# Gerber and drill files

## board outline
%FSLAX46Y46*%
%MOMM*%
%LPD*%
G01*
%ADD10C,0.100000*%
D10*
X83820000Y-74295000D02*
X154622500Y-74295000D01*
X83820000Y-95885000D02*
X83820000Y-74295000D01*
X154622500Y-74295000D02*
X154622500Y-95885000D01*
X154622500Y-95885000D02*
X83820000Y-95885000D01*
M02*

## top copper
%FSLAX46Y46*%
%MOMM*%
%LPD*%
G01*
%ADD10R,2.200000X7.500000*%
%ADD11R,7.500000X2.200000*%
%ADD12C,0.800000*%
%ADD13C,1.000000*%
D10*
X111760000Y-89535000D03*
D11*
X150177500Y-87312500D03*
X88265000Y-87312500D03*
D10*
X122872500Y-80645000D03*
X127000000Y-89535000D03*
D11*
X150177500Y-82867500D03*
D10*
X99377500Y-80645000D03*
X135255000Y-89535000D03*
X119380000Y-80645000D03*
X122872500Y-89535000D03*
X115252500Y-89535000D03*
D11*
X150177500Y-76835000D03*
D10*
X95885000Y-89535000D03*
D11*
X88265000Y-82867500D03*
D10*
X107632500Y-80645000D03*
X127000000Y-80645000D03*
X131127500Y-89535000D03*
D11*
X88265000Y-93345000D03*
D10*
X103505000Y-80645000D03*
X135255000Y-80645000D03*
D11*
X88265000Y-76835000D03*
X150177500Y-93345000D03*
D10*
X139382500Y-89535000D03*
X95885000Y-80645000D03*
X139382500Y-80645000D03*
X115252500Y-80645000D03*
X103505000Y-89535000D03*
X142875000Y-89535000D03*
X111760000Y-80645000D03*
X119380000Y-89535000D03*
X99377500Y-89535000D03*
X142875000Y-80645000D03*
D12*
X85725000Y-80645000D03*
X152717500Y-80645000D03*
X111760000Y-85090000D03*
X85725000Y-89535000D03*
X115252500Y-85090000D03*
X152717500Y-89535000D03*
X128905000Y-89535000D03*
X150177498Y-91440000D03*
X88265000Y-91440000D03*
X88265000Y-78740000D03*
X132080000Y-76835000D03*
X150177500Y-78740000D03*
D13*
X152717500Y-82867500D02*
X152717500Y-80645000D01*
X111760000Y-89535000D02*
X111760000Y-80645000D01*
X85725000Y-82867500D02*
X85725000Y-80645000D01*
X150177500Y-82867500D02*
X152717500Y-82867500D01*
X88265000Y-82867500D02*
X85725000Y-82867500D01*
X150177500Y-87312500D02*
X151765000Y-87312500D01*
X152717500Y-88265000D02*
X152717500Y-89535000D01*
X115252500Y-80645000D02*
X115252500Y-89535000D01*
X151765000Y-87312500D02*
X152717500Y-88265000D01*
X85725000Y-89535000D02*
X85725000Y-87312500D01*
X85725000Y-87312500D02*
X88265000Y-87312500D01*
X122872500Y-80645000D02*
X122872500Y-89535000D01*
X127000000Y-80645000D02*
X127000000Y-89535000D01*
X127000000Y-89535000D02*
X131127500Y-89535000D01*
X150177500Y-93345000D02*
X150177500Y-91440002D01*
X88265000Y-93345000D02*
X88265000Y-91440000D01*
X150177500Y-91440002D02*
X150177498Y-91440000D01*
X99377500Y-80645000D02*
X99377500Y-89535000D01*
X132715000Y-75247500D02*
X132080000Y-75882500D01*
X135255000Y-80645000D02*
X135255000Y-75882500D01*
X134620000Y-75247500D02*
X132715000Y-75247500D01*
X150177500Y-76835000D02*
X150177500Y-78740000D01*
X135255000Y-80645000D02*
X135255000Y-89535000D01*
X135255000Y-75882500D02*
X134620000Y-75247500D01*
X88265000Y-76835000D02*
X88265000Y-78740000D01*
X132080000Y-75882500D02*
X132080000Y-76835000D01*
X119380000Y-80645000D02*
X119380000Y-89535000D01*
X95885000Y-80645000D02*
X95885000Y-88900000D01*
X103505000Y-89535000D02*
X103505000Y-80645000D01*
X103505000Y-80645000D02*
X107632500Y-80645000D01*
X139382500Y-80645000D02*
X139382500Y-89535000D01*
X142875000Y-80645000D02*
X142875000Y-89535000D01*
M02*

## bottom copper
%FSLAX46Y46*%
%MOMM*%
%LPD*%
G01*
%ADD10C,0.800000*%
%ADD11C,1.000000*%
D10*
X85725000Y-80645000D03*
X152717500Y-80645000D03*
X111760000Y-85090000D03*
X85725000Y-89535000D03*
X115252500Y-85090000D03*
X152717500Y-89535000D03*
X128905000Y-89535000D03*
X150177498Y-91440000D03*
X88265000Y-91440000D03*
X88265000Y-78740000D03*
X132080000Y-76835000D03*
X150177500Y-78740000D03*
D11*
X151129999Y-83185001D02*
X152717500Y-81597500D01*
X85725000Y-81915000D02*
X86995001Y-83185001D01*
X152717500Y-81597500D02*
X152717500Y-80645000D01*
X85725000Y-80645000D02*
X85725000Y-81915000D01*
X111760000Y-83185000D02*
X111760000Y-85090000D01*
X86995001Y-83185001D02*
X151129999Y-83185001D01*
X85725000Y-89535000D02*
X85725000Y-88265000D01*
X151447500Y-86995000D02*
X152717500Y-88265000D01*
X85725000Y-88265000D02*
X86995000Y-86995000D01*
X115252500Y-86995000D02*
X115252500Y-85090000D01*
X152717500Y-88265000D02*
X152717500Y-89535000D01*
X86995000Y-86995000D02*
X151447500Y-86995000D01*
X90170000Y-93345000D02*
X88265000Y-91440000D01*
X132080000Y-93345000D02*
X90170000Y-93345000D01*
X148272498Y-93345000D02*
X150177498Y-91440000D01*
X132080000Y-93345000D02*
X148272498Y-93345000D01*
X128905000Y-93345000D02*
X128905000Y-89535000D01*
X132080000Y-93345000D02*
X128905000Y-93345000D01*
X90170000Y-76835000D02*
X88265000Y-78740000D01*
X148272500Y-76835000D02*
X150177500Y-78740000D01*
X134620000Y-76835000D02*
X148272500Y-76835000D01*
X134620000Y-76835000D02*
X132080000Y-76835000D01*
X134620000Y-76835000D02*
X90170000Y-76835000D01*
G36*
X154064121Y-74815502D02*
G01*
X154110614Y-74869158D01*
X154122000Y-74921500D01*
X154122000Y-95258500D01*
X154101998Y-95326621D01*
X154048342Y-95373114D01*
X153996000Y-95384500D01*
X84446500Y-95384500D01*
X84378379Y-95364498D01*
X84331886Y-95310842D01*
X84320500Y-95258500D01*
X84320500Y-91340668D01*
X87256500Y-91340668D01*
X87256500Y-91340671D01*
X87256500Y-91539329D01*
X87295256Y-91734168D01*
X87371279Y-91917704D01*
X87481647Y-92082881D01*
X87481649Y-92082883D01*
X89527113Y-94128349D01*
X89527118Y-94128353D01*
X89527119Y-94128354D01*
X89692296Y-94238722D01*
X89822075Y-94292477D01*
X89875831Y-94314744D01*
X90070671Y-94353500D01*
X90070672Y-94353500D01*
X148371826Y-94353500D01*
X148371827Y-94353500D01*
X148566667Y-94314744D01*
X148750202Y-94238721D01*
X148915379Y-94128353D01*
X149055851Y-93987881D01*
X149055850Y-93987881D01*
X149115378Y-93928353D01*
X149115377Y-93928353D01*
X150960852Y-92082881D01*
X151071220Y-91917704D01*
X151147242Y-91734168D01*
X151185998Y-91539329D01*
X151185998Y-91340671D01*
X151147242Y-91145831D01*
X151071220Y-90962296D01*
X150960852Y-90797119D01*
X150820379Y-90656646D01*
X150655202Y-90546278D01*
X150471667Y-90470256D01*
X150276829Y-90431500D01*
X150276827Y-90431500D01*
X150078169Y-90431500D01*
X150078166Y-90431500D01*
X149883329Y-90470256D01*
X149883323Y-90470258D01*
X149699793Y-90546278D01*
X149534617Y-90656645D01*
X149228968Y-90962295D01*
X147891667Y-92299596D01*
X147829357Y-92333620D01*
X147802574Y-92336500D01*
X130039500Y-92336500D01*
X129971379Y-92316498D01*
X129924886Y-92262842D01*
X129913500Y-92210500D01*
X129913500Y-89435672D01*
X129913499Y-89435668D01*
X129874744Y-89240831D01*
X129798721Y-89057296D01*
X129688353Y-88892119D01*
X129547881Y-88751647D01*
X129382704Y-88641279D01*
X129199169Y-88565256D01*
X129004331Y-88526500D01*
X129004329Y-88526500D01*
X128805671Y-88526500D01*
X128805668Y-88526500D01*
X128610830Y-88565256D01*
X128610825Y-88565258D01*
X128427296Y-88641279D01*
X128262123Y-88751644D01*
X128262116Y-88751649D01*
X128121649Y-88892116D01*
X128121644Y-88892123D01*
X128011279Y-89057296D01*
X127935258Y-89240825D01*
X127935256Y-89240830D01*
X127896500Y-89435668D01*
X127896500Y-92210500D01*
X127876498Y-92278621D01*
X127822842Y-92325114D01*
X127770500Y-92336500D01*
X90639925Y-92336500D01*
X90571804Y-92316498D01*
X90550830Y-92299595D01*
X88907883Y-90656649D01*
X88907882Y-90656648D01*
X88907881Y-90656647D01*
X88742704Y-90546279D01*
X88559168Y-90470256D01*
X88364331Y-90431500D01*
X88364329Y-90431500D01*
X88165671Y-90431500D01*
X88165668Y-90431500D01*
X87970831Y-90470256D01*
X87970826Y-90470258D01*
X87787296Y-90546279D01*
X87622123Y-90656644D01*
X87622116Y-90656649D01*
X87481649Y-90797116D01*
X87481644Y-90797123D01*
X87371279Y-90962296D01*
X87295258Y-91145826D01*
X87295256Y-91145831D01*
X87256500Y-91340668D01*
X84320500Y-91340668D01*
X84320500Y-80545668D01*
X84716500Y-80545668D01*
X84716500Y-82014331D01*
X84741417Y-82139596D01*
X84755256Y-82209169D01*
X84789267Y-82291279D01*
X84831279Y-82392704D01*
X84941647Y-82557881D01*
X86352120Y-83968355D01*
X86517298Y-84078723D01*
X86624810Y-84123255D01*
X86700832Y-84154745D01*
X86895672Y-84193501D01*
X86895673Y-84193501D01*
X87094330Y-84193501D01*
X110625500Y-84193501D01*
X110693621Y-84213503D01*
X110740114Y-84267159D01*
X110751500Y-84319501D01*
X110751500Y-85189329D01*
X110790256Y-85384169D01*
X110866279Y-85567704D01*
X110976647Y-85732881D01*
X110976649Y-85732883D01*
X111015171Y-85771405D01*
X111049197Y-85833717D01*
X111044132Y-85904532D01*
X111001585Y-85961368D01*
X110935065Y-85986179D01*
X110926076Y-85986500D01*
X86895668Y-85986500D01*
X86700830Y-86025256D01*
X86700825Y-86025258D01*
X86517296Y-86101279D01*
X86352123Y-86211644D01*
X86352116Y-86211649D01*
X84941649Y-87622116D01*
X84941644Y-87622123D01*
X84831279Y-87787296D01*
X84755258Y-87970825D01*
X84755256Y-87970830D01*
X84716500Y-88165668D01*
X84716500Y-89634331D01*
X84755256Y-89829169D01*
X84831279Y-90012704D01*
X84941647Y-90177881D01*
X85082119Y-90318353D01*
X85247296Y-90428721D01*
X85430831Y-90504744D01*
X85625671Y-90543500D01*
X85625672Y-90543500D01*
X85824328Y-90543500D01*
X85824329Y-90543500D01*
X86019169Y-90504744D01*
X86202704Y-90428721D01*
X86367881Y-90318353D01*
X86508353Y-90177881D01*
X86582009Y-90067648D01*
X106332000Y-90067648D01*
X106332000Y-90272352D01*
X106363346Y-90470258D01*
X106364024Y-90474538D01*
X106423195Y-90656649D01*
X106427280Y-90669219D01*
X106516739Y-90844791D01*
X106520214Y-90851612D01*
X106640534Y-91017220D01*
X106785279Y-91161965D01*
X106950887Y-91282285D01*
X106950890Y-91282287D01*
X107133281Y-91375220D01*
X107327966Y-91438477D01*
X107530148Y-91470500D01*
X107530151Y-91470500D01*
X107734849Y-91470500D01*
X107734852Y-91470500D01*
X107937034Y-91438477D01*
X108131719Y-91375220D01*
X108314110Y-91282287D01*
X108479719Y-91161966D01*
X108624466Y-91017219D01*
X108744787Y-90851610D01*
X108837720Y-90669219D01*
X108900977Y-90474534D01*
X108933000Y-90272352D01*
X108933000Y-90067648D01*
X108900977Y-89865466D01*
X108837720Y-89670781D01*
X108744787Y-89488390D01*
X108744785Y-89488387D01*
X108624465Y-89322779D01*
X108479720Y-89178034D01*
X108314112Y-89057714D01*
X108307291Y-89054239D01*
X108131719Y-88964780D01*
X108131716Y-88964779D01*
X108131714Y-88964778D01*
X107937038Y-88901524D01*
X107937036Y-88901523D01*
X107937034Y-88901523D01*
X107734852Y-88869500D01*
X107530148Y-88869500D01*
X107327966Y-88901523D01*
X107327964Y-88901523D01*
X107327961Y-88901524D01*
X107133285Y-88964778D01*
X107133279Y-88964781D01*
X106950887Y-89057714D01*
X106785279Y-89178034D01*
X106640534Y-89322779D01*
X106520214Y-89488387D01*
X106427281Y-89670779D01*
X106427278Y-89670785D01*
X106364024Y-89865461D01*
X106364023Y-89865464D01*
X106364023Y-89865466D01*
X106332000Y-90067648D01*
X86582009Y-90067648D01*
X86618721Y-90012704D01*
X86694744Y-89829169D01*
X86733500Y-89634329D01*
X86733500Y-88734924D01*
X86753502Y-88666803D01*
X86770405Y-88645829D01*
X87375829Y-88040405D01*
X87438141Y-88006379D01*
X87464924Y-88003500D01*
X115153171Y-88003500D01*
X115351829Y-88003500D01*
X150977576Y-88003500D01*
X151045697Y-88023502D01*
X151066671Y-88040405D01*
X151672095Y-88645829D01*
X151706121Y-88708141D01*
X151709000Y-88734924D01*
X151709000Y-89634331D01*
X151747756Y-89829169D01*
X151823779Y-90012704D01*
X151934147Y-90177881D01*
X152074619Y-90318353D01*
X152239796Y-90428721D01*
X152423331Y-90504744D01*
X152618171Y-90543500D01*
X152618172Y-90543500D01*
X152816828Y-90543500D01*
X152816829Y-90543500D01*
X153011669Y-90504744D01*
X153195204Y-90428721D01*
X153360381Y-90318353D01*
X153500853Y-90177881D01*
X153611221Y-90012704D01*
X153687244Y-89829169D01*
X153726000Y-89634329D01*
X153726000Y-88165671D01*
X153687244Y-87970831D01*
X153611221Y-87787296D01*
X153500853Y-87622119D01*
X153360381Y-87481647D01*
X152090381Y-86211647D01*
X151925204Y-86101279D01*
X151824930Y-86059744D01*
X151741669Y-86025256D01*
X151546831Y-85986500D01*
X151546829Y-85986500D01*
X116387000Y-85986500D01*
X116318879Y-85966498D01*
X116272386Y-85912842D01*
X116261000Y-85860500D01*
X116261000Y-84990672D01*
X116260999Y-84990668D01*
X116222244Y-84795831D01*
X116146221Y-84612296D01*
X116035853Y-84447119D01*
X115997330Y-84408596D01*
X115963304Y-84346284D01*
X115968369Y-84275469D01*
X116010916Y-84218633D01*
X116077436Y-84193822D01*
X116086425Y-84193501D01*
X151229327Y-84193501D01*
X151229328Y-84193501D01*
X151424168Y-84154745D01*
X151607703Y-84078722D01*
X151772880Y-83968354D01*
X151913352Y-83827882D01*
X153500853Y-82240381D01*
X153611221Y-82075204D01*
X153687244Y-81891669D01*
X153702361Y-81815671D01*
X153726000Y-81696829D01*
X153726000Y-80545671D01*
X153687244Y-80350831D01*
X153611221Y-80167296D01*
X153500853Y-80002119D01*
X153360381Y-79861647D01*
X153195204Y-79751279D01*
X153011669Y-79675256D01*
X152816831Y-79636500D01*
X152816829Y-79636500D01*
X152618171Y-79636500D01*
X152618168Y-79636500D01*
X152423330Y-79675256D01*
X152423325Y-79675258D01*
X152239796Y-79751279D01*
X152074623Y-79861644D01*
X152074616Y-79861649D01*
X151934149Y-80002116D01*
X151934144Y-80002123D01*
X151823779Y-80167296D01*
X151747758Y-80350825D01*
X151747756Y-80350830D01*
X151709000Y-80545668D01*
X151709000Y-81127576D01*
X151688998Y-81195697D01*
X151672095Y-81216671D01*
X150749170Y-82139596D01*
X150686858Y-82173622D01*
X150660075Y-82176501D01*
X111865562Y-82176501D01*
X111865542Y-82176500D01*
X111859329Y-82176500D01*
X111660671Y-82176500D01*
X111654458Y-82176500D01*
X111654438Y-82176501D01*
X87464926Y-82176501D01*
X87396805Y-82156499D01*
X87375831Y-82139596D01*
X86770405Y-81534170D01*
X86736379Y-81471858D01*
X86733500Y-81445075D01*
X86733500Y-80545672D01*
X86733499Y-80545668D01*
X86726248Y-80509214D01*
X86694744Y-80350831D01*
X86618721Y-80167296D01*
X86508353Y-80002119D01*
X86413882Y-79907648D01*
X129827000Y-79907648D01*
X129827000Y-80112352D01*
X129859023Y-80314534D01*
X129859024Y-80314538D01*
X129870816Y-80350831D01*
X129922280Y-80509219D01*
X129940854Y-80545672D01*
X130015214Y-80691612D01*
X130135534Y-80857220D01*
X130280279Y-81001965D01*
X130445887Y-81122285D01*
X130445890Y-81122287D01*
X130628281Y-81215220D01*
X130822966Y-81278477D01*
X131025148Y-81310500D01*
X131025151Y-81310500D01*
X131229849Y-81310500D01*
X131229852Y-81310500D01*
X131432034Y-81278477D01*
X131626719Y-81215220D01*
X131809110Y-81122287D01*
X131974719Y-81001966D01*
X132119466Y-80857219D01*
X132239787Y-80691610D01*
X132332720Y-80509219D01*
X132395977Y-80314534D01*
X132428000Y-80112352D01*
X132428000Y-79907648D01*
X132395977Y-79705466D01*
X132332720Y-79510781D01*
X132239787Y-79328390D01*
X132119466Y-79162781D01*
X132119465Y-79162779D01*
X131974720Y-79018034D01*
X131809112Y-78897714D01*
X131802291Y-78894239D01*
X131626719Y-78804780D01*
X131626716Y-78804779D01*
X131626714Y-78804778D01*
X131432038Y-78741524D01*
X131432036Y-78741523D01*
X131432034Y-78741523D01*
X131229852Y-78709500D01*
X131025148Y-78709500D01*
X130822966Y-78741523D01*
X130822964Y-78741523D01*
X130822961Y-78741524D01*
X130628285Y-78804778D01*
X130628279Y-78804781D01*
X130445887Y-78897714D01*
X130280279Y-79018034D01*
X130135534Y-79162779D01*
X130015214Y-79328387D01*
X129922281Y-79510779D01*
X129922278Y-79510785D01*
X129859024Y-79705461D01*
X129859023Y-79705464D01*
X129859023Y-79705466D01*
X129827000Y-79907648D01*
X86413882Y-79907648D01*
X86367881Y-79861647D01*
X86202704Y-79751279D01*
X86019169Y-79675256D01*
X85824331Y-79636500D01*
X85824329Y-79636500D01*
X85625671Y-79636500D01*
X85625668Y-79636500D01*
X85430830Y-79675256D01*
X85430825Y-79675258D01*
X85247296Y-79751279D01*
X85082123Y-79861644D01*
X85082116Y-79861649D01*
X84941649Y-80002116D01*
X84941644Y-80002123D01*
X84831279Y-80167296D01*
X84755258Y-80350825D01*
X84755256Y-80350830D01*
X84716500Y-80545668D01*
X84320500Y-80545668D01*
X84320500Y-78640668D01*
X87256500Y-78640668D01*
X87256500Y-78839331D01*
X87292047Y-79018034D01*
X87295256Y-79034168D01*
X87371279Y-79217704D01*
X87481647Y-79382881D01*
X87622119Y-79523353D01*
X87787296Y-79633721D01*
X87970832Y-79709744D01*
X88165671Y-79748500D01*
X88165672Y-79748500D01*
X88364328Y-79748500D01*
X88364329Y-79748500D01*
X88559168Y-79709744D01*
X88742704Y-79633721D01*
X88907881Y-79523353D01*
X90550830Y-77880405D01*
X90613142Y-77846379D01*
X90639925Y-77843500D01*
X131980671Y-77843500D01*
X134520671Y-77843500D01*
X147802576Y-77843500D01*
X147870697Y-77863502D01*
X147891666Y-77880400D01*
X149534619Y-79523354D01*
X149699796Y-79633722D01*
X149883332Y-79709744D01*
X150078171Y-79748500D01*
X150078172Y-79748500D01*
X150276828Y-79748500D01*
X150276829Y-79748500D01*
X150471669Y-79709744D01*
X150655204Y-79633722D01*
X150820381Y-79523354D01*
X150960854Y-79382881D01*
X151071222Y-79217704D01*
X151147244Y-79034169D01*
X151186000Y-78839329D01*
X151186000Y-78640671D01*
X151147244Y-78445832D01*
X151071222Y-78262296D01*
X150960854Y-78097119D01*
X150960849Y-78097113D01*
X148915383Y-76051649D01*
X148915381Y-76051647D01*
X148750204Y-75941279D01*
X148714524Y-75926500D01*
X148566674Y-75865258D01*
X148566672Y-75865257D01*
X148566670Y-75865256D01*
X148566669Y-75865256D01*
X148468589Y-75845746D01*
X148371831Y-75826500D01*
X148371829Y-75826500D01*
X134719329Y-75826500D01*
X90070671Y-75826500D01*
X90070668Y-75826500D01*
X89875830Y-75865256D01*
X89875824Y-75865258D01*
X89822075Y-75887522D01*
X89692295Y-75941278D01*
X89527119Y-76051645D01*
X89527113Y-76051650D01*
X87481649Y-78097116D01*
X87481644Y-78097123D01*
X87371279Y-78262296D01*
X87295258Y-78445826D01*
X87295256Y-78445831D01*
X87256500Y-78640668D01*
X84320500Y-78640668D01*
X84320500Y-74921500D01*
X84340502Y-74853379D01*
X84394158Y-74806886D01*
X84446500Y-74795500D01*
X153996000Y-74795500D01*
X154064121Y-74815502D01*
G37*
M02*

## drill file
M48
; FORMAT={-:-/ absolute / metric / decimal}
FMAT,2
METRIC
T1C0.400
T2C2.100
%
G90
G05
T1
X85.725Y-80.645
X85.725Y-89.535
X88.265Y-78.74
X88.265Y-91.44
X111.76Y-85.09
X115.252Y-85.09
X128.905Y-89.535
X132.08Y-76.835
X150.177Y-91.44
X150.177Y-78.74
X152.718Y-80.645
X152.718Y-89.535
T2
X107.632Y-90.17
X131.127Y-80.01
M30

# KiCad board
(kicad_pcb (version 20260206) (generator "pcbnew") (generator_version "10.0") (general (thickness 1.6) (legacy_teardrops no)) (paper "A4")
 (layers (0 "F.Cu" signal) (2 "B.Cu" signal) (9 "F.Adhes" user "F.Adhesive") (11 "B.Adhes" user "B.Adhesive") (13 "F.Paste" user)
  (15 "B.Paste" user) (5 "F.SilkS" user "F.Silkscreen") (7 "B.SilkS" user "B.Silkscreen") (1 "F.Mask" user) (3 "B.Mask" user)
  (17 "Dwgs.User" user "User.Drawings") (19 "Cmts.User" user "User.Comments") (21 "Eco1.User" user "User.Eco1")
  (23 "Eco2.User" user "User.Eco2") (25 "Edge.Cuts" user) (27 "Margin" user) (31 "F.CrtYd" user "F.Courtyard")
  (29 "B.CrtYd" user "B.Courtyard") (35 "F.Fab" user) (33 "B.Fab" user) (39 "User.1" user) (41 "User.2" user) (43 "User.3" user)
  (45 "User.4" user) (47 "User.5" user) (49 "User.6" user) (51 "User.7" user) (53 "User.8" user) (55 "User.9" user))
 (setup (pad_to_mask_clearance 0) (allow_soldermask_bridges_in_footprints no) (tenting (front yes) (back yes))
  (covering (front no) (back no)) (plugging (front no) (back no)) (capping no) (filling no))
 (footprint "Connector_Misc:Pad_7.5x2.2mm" (layer "F.Cu") (at 111.76 89.535 -90)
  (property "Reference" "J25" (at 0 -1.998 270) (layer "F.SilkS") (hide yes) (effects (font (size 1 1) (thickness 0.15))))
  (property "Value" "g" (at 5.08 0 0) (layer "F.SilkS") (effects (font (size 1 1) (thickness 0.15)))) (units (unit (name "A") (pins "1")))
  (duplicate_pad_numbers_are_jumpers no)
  (pad "1" smd rect (at 0 0 270) (size 7.5 2.2) (layers "F.Cu" "F.Mask") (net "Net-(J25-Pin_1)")))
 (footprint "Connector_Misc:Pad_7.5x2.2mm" (layer "F.Cu") (at 150.1775 87.3125)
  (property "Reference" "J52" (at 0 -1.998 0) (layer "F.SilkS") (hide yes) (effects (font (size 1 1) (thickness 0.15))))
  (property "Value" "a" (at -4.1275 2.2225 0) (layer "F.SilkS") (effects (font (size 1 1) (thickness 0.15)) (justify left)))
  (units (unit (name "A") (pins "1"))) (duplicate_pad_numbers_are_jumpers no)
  (pad "1" smd rect (at 0 0) (size 7.5 2.2) (layers "F.Cu" "F.Mask") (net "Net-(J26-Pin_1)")))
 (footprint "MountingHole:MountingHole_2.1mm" (layer "F.Cu") (at 107.6325 90.17)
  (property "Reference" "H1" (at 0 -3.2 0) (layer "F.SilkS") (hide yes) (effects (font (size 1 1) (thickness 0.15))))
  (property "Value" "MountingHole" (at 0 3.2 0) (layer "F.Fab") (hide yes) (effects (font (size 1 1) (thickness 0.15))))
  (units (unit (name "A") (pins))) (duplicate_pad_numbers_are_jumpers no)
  (pad "" np_thru_hole circle (at 0 0) (size 2.1 2.1) (drill 2.1) (layers "*.Cu" "*.Mask")))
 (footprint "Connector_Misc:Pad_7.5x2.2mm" (layer "F.Cu") (at 88.265 87.3125 180)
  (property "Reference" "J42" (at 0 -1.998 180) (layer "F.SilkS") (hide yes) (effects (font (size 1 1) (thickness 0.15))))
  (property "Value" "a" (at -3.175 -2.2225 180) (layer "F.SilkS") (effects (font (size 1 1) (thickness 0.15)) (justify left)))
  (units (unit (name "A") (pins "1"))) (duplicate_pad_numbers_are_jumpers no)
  (pad "1" smd rect (at 0 0 180) (size 7.5 2.2) (layers "F.Cu" "F.Mask") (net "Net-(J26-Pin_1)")))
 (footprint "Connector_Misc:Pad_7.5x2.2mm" (layer "F.Cu") (at 122.8725 80.645 90)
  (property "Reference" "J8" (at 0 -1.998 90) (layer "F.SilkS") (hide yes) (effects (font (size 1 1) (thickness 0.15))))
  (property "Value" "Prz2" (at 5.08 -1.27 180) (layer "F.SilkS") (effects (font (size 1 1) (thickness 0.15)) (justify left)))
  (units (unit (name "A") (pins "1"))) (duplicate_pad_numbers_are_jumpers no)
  (pad "1" smd rect (at 0 0 90) (size 7.5 2.2) (layers "F.Cu" "F.Mask") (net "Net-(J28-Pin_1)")))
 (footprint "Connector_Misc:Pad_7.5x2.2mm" (layer "F.Cu") (at 127 89.535 -90)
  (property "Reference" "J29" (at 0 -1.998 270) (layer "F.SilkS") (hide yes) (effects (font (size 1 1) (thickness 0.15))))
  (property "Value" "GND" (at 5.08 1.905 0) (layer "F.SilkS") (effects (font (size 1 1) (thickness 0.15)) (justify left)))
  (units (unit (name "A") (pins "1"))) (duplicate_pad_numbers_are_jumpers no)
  (pad "1" smd rect (at 0 0 270) (size 7.5 2.2) (layers "F.Cu" "F.Mask") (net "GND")))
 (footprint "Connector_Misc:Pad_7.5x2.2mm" (layer "F.Cu") (at 150.1775 82.8675)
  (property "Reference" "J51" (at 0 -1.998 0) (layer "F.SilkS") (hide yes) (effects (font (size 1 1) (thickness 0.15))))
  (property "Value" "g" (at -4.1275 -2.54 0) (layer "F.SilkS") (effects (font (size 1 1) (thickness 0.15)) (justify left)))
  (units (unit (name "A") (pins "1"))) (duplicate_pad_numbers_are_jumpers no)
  (pad "1" smd rect (at 0 0) (size 7.5 2.2) (layers "F.Cu" "F.Mask") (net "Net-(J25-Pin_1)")))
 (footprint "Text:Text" (layer "F.Cu") (at 102.743 79.883)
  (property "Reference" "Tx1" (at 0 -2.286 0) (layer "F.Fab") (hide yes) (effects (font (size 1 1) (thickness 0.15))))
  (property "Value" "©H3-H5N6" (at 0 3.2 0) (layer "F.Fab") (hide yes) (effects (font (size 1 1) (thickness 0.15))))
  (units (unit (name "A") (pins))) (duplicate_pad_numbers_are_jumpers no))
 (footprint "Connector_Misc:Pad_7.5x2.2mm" (layer "F.Cu") (at 99.3775 80.645 90)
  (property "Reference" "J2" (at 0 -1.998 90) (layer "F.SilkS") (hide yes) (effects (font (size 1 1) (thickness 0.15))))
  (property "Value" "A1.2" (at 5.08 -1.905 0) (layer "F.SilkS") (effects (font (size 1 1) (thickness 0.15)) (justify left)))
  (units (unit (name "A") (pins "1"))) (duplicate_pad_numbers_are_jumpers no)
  (pad "1" smd rect (at 0 0 90) (size 7.5 2.2) (layers "F.Cu" "F.Mask") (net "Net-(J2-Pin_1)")))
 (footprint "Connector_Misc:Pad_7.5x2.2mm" (layer "F.Cu") (at 135.255 89.535 90)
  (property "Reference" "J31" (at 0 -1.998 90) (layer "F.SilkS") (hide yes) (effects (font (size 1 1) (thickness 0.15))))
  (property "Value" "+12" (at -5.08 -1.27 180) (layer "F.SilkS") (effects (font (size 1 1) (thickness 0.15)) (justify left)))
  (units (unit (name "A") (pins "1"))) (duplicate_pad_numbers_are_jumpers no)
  (pad "1" smd rect (at 0 0 90) (size 7.5 2.2) (layers "F.Cu" "F.Mask") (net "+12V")))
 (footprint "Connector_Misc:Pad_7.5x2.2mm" (layer "F.Cu") (at 119.38 80.645 90)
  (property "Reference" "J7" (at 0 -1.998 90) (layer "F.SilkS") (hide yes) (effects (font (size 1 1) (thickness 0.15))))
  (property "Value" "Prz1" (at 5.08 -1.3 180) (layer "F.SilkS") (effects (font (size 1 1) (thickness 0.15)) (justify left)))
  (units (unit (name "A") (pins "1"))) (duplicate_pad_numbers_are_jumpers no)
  (pad "1" smd rect (at 0 0 90) (size 7.5 2.2) (layers "F.Cu" "F.Mask") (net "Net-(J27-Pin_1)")))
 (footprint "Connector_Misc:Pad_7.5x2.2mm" (layer "F.Cu") (at 122.8725 89.535 -90)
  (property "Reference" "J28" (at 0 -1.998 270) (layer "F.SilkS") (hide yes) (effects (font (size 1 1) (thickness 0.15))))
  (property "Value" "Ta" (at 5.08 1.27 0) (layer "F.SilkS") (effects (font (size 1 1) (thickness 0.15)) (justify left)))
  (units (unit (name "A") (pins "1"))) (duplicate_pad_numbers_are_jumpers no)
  (pad "1" smd rect (at 0 0 270) (size 7.5 2.2) (layers "F.Cu" "F.Mask") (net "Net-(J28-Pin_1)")))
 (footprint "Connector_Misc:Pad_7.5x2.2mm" (layer "F.Cu") (at 115.2525 89.535 -90)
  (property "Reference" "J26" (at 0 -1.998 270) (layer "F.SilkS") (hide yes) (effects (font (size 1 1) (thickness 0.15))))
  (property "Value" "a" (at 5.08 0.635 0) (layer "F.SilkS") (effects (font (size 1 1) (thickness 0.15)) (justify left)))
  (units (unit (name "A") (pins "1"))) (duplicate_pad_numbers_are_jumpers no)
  (pad "1" smd rect (at 0 0 270) (size 7.5 2.2) (layers "F.Cu" "F.Mask") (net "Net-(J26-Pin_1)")))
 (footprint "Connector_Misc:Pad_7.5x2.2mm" (layer "F.Cu") (at 150.1775 76.835 180)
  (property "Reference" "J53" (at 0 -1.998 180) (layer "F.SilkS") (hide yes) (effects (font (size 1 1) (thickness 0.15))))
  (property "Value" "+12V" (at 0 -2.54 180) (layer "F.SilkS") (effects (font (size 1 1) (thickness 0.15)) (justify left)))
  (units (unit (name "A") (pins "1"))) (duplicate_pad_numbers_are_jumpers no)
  (pad "1" smd rect (at 0 0 180) (size 7.5 2.2) (layers "F.Cu" "F.Mask") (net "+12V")))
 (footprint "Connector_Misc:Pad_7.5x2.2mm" (layer "F.Cu") (at 95.885 89.535 -90)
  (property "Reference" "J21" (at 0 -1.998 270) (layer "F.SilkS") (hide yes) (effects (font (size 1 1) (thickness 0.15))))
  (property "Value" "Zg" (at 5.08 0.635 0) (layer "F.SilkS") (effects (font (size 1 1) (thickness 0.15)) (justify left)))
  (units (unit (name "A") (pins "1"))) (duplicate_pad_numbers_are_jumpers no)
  (pad "1" smd rect (at 0 0 270) (size 7.5 2.2) (layers "F.Cu" "F.Mask") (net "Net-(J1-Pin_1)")))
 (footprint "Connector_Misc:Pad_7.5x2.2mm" (layer "F.Cu") (at 88.265 82.8675 180)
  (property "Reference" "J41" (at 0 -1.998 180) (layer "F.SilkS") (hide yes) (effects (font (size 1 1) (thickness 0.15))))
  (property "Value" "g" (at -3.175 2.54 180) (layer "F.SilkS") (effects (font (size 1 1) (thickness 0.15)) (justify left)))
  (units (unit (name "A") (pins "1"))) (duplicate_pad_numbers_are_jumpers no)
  (pad "1" smd rect (at 0 0 180) (size 7.5 2.2) (layers "F.Cu" "F.Mask") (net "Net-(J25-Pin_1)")))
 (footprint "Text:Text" (layer "F.Cu") (at 124.587 89.535)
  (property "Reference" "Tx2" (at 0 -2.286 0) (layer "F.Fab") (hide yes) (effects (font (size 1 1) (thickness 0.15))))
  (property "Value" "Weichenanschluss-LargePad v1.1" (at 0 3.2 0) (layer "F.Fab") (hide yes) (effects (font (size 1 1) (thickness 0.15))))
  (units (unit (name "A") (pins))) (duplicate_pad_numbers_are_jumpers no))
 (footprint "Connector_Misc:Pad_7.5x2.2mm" (layer "F.Cu") (at 107.6325 80.645 90)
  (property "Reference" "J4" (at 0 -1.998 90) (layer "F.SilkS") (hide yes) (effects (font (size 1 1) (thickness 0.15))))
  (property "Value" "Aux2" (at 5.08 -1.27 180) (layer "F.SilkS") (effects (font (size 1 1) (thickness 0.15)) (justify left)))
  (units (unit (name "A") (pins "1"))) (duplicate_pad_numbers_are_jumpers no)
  (pad "1" smd rect (at 0 0 90) (size 7.5 2.2) (layers "F.Cu" "F.Mask") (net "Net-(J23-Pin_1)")))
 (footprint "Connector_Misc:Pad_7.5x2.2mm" (layer "F.Cu") (at 127 80.645 90)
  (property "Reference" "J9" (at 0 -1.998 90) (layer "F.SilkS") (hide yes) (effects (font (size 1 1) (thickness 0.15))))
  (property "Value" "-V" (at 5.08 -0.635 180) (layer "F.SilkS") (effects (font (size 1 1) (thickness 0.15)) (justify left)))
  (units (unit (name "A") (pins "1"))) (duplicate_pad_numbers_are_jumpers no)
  (pad "1" smd rect (at 0 0 90) (size 7.5 2.2) (layers "F.Cu" "F.Mask") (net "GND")))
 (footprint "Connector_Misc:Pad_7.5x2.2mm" (layer "F.Cu") (at 131.1275 89.535 -90)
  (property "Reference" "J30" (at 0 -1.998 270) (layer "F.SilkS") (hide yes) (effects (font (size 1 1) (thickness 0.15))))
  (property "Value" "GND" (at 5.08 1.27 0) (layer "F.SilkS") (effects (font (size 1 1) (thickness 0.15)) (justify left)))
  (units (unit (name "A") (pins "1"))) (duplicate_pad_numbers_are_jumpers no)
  (pad "1" smd rect (at 0 0 270) (size 7.5 2.2) (layers "F.Cu" "F.Mask") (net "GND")))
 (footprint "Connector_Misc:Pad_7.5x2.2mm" (layer "F.Cu") (at 88.265 93.345)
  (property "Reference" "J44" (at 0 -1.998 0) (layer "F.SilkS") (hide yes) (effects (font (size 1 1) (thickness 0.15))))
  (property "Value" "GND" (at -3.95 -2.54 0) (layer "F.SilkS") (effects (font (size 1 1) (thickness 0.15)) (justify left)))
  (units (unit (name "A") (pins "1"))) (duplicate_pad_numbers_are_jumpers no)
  (pad "1" smd rect (at 0 0) (size 7.5 2.2) (layers "F.Cu" "F.Mask") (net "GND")))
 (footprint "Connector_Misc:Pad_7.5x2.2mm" (layer "F.Cu") (at 103.505 80.645 90)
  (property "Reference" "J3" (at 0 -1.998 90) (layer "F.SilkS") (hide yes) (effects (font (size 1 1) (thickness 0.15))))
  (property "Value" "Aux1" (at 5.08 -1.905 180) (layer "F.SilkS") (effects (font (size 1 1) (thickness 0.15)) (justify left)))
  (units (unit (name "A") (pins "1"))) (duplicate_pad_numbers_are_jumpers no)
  (pad "1" smd rect (at 0 0 90) (size 7.5 2.2) (layers "F.Cu" "F.Mask") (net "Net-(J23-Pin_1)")))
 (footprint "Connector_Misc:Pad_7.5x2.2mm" (layer "F.Cu") (at 135.255 80.645 90)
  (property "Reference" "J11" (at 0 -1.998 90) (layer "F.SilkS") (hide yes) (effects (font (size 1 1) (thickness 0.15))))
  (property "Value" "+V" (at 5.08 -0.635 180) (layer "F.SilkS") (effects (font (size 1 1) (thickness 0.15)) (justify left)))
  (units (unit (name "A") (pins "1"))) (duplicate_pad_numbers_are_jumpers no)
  (pad "1" smd rect (at 0 0 90) (size 7.5 2.2) (layers "F.Cu" "F.Mask") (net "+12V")))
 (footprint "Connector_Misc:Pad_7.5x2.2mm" (layer "F.Cu") (at 88.265 76.835)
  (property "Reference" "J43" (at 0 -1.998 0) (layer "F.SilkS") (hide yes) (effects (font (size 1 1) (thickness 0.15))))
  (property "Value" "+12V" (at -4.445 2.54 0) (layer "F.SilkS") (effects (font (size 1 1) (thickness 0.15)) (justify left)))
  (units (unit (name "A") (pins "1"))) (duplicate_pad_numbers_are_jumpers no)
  (pad "1" smd rect (at 0 0) (size 7.5 2.2) (layers "F.Cu" "F.Mask") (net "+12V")))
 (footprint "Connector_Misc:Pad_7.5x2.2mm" (layer "F.Cu") (at 150.1775 93.345)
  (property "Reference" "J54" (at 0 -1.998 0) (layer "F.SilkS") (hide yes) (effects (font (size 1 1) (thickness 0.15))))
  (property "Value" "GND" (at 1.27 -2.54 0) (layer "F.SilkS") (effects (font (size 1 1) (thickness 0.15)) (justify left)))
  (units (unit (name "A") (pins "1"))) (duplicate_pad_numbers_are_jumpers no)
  (pad "1" smd rect (at 0 0) (size 7.5 2.2) (layers "F.Cu" "F.Mask") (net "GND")))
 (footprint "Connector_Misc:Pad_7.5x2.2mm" (layer "F.Cu") (at 139.3825 89.535 90)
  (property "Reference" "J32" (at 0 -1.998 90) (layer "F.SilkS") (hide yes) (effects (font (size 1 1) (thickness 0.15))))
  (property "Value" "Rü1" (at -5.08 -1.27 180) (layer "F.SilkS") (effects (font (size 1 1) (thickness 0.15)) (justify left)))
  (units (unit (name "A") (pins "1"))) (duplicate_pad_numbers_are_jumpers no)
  (pad "1" smd rect (at 0 0 90) (size 7.5 2.2) (layers "F.Cu" "F.Mask") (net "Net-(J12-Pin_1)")))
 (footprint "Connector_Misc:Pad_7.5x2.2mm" (layer "F.Cu") (at 95.885 80.645 90)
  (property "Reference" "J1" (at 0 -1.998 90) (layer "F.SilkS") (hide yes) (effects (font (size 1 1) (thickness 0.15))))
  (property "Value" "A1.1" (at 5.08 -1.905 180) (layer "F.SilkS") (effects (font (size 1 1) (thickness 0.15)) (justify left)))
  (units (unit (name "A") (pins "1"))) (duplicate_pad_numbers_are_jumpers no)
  (pad "1" smd rect (at 0 0 90) (size 7.5 2.2) (layers "F.Cu" "F.Mask") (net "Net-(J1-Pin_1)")))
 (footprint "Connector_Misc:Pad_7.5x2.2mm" (layer "F.Cu") (at 139.3825 80.645 90)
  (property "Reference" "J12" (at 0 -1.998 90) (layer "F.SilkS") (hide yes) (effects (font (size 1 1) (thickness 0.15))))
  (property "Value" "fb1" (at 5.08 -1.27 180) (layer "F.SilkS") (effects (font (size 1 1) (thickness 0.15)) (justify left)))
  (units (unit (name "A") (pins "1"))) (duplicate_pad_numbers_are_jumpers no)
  (pad "1" smd rect (at 0 0 90) (size 7.5 2.2) (layers "F.Cu" "F.Mask") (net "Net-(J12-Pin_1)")))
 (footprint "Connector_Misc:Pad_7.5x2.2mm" (layer "F.Cu") (at 115.2525 80.645 90)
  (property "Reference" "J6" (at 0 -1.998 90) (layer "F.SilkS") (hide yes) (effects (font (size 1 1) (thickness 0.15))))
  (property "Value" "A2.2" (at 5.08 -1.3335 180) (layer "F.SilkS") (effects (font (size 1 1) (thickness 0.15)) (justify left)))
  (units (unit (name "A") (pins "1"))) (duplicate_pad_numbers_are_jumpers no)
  (pad "1" smd rect (at 0 0 90) (size 7.5 2.2) (layers "F.Cu" "F.Mask") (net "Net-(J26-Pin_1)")))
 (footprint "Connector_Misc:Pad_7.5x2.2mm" (layer "F.Cu") (at 103.505 89.535 -90)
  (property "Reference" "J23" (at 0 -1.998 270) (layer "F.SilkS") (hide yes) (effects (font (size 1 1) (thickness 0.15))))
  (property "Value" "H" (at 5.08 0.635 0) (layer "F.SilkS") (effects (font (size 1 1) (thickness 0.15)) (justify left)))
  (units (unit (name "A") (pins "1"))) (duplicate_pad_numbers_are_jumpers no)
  (pad "1" smd rect (at 0 0 270) (size 7.5 2.2) (layers "F.Cu" "F.Mask") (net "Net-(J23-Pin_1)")))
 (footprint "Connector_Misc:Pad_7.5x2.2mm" (layer "F.Cu") (at 142.875 89.535 90)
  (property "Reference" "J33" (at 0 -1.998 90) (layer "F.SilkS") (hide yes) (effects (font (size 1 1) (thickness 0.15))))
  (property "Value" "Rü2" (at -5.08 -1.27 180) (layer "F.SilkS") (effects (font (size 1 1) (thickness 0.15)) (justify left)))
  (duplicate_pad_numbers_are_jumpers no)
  (pad "1" smd rect (at 0 0 90) (size 7.5 2.2) (layers "F.Cu" "F.Mask") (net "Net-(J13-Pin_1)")))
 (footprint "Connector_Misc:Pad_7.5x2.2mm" (layer "F.Cu") (at 111.76 80.645 90)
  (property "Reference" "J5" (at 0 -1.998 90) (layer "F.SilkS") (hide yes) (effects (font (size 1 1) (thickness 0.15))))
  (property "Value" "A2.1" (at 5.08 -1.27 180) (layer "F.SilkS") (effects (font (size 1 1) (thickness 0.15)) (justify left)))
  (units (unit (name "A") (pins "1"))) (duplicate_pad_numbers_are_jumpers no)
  (pad "1" smd rect (at 0 0 90) (size 7.5 2.2) (layers "F.Cu" "F.Mask") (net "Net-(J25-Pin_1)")))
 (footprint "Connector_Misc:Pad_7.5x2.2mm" (layer "F.Cu") (at 119.38 89.535 -90)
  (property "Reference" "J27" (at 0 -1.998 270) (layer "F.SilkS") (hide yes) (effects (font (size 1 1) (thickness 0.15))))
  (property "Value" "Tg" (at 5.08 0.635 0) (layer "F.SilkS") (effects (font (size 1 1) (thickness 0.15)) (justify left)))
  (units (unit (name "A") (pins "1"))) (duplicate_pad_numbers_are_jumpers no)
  (pad "1" smd rect (at 0 0 270) (size 7.5 2.2) (layers "F.Cu" "F.Mask") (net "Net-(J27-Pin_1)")))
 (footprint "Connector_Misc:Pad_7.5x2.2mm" (layer "F.Cu") (at 99.3775 89.535 -90)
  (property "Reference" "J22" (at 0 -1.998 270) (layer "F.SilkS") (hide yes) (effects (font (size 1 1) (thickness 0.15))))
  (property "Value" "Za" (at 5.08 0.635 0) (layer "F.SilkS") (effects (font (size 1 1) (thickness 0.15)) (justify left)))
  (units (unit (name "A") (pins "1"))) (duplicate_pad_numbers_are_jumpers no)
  (pad "1" smd rect (at 0 0 270) (size 7.5 2.2) (layers "F.Cu" "F.Mask") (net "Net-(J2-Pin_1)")))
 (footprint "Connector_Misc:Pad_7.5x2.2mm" (layer "F.Cu") (at 142.875 80.645 90)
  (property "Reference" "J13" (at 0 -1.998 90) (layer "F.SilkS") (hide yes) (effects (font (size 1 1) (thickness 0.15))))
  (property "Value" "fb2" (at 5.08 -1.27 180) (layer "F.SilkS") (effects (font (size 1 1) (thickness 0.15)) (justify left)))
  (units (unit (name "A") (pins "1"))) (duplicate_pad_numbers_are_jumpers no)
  (pad "1" smd rect (at 0 0 90) (size 7.5 2.2) (layers "F.Cu" "F.Mask") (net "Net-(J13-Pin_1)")))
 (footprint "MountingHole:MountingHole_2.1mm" (layer "F.Cu") (at 131.1275 80.01)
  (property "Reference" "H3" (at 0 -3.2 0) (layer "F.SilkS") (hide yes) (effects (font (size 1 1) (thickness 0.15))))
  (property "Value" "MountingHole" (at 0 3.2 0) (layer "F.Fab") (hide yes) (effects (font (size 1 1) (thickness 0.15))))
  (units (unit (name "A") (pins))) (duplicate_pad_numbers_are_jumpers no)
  (pad "" np_thru_hole circle (at 0 0) (size 2.1 2.1) (drill 2.1) (layers "*.Cu" "*.Mask")))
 (gr_line (start 83.82 74.295) (end 154.6225 74.295) (stroke (width 0.1) (type solid)) (layer "Edge.Cuts"))
 (gr_line (start 83.82 95.885) (end 83.82 74.295) (stroke (width 0.1) (type solid)) (layer "Edge.Cuts"))
 (gr_line (start 154.6225 74.295) (end 154.6225 95.885) (stroke (width 0.1) (type solid)) (layer "Edge.Cuts"))
 (gr_line (start 154.6225 95.885) (end 83.82 95.885) (stroke (width 0.1) (type solid)) (layer "Edge.Cuts"))
 (segment (start 152.7175 82.8675) (end 152.7175 80.645) (width 1) (layer "F.Cu") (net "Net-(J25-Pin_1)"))
 (segment (start 111.76 89.535) (end 111.76 80.645) (width 1) (layer "F.Cu") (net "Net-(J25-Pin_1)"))
 (segment (start 85.725 82.8675) (end 85.725 80.645) (width 1) (layer "F.Cu") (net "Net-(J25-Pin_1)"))
 (segment (start 150.1775 82.8675) (end 152.7175 82.8675) (width 1) (layer "F.Cu") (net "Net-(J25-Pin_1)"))
 (segment (start 88.265 82.8675) (end 85.725 82.8675) (width 1) (layer "F.Cu") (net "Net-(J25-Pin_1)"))
 (via (at 85.725 80.645) (size 0.8) (drill 0.4) (layers "F.Cu" "B.Cu") (capping no) (covering (front no) (back no))
  (plugging (front no) (back no)) (filling no) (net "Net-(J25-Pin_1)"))
 (via (at 152.7175 80.645) (size 0.8) (drill 0.4) (layers "F.Cu" "B.Cu") (capping no) (covering (front no) (back no))
  (plugging (front no) (back no)) (filling no) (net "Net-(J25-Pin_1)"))
 (via (at 111.76 85.09) (size 0.8) (drill 0.4) (layers "F.Cu" "B.Cu") (capping no) (covering (front no) (back no))
  (plugging (front no) (back no)) (filling no) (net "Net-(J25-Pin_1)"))
 (segment (start 151.129999 83.185001) (end 152.7175 81.5975) (width 1) (layer "B.Cu") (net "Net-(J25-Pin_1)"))
 (segment (start 85.725 81.915) (end 86.995001 83.185001) (width 1) (layer "B.Cu") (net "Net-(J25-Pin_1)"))
 (segment (start 152.7175 81.5975) (end 152.7175 80.645) (width 1) (layer "B.Cu") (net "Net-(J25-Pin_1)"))
 (segment (start 85.725 80.645) (end 85.725 81.915) (width 1) (layer "B.Cu") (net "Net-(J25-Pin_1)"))
 (segment (start 111.76 83.185) (end 111.76 85.09) (width 1) (layer "B.Cu") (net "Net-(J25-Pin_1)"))
 (segment (start 86.995001 83.185001) (end 151.129999 83.185001) (width 1) (layer "B.Cu") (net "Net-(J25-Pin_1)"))
 (segment (start 150.1775 87.3125) (end 151.765 87.3125) (width 1) (layer "F.Cu") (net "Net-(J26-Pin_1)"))
 (segment (start 152.7175 88.265) (end 152.7175 89.535) (width 1) (layer "F.Cu") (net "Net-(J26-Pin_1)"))
 (segment (start 115.2525 80.645) (end 115.2525 89.535) (width 1) (layer "F.Cu") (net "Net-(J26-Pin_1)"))
 (segment (start 151.765 87.3125) (end 152.7175 88.265) (width 1) (layer "F.Cu") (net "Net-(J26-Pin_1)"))
 (segment (start 85.725 89.535) (end 85.725 87.3125) (width 1) (layer "F.Cu") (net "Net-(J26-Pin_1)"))
 (segment (start 85.725 87.3125) (end 88.265 87.3125) (width 1) (layer "F.Cu") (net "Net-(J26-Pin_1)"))
 (via (at 85.725 89.535) (size 0.8) (drill 0.4) (layers "F.Cu" "B.Cu") (capping no) (covering (front no) (back no))
  (plugging (front no) (back no)) (filling no) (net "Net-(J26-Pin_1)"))
 (via (at 115.2525 85.09) (size 0.8) (drill 0.4) (layers "F.Cu" "B.Cu") (capping no) (covering (front no) (back no))
  (plugging (front no) (back no)) (filling no) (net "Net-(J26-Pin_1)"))
 (via (at 152.7175 89.535) (size 0.8) (drill 0.4) (layers "F.Cu" "B.Cu") (capping no) (covering (front no) (back no))
  (plugging (front no) (back no)) (filling no) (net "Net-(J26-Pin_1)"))
 (segment (start 85.725 89.535) (end 85.725 88.265) (width 1) (layer "B.Cu") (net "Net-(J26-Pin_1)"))
 (segment (start 151.4475 86.995) (end 152.7175 88.265) (width 1) (layer "B.Cu") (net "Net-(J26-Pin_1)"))
 (segment (start 85.725 88.265) (end 86.995 86.995) (width 1) (layer "B.Cu") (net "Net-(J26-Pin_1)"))
 (segment (start 115.2525 86.995) (end 115.2525 85.09) (width 1) (layer "B.Cu") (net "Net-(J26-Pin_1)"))
 (segment (start 152.7175 88.265) (end 152.7175 89.535) (width 1) (layer "B.Cu") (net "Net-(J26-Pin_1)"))
 (segment (start 86.995 86.995) (end 151.4475 86.995) (width 1) (layer "B.Cu") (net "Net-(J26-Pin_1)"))
 (segment (start 122.8725 80.645) (end 122.8725 89.535) (width 1) (layer "F.Cu") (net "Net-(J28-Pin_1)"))
 (segment (start 127 80.645) (end 127 89.535) (width 1) (layer "F.Cu") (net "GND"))
 (segment (start 127 89.535) (end 131.1275 89.535) (width 1) (layer "F.Cu") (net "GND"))
 (segment (start 150.1775 93.345) (end 150.1775 91.440002) (width 1) (layer "F.Cu") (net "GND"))
 (segment (start 88.265 93.345) (end 88.265 91.44) (width 1) (layer "F.Cu") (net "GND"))
 (segment (start 150.1775 91.440002) (end 150.177498 91.44) (width 1) (layer "F.Cu") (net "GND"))
 (via (at 128.905 89.535) (size 0.8) (drill 0.4) (layers "F.Cu" "B.Cu") (capping no) (covering (front no) (back no))
  (plugging (front no) (back no)) (filling no) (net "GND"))
 (via (at 150.177498 91.44) (size 0.8) (drill 0.4) (layers "F.Cu" "B.Cu") (capping no) (covering (front no) (back no))
  (plugging (front no) (back no)) (filling no) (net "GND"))
 (via (at 88.265 91.44) (size 0.8) (drill 0.4) (layers "F.Cu" "B.Cu") (capping no) (covering (front no) (back no))
  (plugging (front no) (back no)) (filling no) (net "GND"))
 (segment (start 90.17 93.345) (end 88.265 91.44) (width 1) (layer "B.Cu") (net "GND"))
 (segment (start 132.08 93.345) (end 90.17 93.345) (width 1) (layer "B.Cu") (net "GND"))
 (segment (start 148.272498 93.345) (end 150.177498 91.44) (width 1) (layer "B.Cu") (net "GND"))
 (segment (start 132.08 93.345) (end 148.272498 93.345) (width 1) (layer "B.Cu") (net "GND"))
 (segment (start 128.905 93.345) (end 128.905 89.535) (width 1) (layer "B.Cu") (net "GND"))
 (segment (start 132.08 93.345) (end 128.905 93.345) (width 1) (layer "B.Cu") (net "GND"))
 (segment (start 99.3775 80.645) (end 99.3775 89.535) (width 1) (layer "F.Cu") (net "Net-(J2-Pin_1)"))
 (segment (start 132.715 75.2475) (end 132.08 75.8825) (width 1) (layer "F.Cu") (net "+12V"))
 (segment (start 135.255 80.645) (end 135.255 75.8825) (width 1) (layer "F.Cu") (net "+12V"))
 (segment (start 134.62 75.2475) (end 132.715 75.2475) (width 1) (layer "F.Cu") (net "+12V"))
 (segment (start 150.1775 76.835) (end 150.1775 78.74) (width 1) (layer "F.Cu") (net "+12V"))
 (segment (start 135.255 80.645) (end 135.255 89.535) (width 1) (layer "F.Cu") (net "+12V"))
 (segment (start 135.255 75.8825) (end 134.62 75.2475) (width 1) (layer "F.Cu") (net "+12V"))
 (segment (start 88.265 76.835) (end 88.265 78.74) (width 1) (layer "F.Cu") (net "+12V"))
 (segment (start 132.08 75.8825) (end 132.08 76.835) (width 1) (layer "F.Cu") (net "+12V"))
 (via (at 88.265 78.74) (size 0.8) (drill 0.4) (layers "F.Cu" "B.Cu") (capping no) (covering (front no) (back no))
  (plugging (front no) (back no)) (filling no) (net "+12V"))
 (via (at 132.08 76.835) (size 0.8) (drill 0.4) (layers "F.Cu" "B.Cu") (capping no) (covering (front no) (back no))
  (plugging (front no) (back no)) (filling no) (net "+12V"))
 (via (at 150.1775 78.74) (size 0.8) (drill 0.4) (layers "F.Cu" "B.Cu") (capping no) (covering (front no) (back no))
  (plugging (front no) (back no)) (filling no) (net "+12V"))
 (segment (start 90.17 76.835) (end 88.265 78.74) (width 1) (layer "B.Cu") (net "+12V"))
 (segment (start 148.2725 76.835) (end 150.1775 78.74) (width 1) (layer "B.Cu") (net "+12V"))
 (segment (start 134.62 76.835) (end 148.2725 76.835) (width 1) (layer "B.Cu") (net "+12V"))
 (segment (start 134.62 76.835) (end 132.08 76.835) (width 1) (layer "B.Cu") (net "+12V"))
 (segment (start 134.62 76.835) (end 90.17 76.835) (width 1) (layer "B.Cu") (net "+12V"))
 (segment (start 119.38 80.645) (end 119.38 89.535) (width 1) (layer "F.Cu") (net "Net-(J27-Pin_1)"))
 (segment (start 95.885 80.645) (end 95.885 88.9) (width 1) (layer "F.Cu") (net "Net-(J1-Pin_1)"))
 (segment (start 103.505 89.535) (end 103.505 80.645) (width 1) (layer "F.Cu") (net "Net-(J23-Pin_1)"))
 (segment (start 103.505 80.645) (end 107.6325 80.645) (width 1) (layer "F.Cu") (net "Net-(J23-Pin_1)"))
 (segment (start 139.3825 80.645) (end 139.3825 89.535) (width 1) (layer "F.Cu") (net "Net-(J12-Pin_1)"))
 (segment (start 142.875 80.645) (end 142.875 89.535) (width 1) (layer "F.Cu") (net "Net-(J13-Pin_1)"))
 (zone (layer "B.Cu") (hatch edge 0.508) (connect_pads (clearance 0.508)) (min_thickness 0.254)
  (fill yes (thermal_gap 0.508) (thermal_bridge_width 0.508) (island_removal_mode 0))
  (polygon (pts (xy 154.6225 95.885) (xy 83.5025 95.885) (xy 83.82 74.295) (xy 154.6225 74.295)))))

